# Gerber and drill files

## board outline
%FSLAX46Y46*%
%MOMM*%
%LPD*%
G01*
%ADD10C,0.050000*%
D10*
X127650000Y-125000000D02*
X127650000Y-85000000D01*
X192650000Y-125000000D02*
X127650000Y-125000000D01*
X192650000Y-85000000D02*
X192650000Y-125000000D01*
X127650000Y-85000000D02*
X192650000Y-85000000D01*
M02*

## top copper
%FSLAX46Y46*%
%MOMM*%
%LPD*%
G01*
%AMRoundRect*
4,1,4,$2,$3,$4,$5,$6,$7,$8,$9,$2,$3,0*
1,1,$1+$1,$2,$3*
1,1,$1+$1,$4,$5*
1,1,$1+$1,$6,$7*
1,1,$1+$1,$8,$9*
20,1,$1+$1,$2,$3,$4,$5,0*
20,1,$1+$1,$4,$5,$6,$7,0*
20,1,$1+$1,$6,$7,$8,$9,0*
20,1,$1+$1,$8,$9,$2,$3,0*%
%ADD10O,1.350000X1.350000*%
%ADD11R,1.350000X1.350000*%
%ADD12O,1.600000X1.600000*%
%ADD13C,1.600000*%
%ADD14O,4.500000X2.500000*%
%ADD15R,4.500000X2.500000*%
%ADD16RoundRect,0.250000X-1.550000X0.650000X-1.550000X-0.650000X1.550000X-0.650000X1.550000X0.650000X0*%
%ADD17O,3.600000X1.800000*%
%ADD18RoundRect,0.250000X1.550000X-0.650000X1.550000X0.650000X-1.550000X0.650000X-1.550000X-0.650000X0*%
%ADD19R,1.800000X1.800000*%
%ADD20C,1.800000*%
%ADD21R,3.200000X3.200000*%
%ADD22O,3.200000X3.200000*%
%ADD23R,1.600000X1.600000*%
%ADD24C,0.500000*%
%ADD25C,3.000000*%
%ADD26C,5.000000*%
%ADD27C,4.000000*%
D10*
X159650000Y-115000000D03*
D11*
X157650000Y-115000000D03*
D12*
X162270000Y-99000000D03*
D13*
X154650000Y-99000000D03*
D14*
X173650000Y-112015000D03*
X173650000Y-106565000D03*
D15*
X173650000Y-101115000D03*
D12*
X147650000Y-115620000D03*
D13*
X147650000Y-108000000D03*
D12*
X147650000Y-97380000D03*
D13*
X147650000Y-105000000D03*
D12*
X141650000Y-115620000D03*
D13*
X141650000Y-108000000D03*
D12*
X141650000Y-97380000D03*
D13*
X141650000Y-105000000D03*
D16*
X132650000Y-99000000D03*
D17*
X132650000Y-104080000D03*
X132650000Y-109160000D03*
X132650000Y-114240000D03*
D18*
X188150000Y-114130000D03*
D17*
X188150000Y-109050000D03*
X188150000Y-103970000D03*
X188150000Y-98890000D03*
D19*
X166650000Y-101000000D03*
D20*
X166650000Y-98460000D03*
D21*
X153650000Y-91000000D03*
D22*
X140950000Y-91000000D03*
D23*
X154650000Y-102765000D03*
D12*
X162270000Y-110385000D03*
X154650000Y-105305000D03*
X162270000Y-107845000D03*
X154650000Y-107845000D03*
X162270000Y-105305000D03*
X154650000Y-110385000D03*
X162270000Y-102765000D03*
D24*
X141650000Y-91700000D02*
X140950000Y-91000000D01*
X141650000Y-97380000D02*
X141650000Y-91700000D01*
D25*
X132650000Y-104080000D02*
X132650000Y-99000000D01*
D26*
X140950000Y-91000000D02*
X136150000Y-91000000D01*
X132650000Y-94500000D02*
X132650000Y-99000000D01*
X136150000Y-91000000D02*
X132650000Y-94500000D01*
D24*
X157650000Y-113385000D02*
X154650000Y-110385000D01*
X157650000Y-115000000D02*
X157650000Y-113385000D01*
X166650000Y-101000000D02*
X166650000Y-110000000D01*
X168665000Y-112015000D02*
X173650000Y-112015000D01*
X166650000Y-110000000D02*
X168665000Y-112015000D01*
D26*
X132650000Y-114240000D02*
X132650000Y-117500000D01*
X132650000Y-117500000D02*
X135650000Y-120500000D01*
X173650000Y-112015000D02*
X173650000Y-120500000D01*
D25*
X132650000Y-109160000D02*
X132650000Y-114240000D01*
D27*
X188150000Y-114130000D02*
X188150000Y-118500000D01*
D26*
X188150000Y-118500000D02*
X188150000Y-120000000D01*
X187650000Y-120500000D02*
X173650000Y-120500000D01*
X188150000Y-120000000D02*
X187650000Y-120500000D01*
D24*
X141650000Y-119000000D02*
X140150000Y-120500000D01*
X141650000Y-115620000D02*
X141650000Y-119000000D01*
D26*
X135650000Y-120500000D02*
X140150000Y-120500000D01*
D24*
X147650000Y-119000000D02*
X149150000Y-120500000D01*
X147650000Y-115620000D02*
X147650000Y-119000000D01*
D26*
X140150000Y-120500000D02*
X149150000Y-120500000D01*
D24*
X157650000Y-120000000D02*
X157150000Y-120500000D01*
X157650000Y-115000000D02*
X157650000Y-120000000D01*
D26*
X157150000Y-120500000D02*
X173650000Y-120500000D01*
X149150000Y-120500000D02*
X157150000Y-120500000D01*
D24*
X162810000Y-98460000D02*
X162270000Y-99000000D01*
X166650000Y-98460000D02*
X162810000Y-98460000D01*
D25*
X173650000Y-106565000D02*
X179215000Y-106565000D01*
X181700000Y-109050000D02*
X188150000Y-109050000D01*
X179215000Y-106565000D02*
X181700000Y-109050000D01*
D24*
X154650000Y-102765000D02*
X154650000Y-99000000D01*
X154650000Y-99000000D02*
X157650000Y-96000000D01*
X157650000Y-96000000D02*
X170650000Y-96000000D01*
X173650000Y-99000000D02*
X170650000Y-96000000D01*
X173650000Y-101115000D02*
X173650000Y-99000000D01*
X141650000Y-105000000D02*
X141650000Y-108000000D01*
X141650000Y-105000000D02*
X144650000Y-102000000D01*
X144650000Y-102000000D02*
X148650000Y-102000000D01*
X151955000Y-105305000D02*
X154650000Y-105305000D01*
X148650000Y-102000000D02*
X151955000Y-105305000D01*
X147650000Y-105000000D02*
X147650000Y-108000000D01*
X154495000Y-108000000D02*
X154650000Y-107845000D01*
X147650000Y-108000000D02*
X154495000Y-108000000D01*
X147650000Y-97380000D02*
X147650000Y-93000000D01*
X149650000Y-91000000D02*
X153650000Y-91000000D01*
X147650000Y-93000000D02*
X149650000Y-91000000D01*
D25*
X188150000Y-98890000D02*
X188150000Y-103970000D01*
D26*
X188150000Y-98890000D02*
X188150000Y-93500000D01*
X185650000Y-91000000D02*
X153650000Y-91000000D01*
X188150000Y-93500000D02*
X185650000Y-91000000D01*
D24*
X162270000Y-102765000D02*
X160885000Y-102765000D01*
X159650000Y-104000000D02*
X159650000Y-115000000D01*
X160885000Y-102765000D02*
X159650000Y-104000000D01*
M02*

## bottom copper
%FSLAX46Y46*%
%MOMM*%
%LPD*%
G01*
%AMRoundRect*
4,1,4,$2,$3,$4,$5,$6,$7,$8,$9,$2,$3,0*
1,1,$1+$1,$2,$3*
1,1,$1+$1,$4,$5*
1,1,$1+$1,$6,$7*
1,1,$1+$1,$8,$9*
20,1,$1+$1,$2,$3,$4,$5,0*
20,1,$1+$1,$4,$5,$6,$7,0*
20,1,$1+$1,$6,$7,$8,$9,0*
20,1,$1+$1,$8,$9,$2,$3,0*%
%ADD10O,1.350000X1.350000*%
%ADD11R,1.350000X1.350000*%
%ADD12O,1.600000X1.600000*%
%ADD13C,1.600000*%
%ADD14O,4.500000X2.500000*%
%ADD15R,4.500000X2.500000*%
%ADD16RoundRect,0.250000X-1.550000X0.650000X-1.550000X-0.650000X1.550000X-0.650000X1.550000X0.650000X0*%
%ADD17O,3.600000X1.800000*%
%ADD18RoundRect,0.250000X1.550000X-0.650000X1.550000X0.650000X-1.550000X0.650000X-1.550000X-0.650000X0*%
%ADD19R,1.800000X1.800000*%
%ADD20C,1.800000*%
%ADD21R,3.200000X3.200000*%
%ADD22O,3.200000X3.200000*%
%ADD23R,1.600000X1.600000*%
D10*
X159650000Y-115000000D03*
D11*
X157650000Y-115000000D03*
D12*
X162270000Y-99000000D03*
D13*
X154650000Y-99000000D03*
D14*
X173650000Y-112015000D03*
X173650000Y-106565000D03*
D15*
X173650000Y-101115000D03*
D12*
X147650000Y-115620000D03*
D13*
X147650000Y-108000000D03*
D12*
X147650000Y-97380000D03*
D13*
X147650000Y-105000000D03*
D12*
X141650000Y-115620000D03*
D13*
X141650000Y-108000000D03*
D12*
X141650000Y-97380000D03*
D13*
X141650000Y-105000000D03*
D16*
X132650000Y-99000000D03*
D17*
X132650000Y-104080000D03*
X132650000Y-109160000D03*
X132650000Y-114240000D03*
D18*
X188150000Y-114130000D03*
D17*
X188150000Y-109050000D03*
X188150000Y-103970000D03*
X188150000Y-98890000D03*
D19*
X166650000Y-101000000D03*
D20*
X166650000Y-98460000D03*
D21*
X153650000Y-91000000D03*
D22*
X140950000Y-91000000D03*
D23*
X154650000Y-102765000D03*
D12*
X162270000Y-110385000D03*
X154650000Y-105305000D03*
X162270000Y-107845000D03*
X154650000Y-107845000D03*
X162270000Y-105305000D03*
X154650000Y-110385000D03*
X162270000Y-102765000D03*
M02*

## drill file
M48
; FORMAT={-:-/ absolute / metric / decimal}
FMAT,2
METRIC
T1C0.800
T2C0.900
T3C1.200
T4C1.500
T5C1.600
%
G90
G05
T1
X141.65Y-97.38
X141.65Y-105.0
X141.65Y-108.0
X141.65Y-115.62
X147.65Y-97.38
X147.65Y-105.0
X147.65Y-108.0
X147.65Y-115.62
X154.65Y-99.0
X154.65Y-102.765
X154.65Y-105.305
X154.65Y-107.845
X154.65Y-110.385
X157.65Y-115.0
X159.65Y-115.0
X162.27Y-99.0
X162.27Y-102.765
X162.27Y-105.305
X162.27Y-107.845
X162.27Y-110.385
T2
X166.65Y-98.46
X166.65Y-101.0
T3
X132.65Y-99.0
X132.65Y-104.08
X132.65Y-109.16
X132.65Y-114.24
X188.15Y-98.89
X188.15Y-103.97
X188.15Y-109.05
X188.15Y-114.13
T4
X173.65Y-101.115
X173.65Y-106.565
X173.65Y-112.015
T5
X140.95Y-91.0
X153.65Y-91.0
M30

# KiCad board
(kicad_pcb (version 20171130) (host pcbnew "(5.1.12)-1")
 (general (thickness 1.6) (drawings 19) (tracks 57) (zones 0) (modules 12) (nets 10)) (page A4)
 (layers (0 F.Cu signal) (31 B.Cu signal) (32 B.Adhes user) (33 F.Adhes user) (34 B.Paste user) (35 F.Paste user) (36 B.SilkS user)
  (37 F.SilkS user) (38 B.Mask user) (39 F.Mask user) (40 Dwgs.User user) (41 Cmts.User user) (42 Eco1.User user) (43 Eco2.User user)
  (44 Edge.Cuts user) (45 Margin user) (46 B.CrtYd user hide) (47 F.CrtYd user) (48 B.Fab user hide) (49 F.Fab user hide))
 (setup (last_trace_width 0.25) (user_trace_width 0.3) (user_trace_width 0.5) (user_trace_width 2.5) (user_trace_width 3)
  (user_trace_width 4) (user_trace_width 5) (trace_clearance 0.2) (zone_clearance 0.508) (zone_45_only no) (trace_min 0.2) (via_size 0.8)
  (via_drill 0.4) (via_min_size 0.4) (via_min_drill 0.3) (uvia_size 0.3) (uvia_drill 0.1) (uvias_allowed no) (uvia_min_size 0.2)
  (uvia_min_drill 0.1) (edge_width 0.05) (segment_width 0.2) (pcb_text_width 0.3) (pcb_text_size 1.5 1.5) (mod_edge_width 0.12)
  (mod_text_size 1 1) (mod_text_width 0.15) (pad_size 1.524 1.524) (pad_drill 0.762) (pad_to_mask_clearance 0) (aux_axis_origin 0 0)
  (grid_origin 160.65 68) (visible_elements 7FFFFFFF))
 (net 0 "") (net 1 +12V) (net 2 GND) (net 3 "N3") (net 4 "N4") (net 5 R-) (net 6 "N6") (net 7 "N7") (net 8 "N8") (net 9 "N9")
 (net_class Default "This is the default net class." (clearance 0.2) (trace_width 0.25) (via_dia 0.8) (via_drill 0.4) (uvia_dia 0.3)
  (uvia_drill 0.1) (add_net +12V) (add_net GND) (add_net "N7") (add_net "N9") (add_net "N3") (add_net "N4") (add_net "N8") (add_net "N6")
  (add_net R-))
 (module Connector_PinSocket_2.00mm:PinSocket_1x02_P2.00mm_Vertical (layer F.Cu) (at 157.65 115 90)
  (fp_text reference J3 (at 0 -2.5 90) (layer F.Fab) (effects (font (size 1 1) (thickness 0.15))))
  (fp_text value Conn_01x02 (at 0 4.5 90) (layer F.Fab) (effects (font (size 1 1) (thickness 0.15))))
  (pad 2 thru_hole oval (at 0 2 90) (size 1.35 1.35) (drill 0.8) (layers *.Cu *.Mask) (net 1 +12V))
  (pad 1 thru_hole rect (at 0 0 90) (size 1.35 1.35) (drill 0.8) (layers *.Cu *.Mask) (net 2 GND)))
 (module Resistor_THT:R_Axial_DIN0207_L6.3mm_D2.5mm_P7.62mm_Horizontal (layer F.Cu) (at 154.65 99)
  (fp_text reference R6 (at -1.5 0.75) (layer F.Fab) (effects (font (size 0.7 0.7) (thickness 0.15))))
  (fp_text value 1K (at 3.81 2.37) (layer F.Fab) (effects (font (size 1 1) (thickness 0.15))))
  (pad 2 thru_hole oval (at 7.62 0) (size 1.6 1.6) (drill 0.8) (layers *.Cu *.Mask) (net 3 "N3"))
  (pad 1 thru_hole circle (at 0 0) (size 1.6 1.6) (drill 0.8) (layers *.Cu *.Mask) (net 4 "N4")))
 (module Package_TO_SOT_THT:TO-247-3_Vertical (layer F.Cu) (at 173.65 101.115 270)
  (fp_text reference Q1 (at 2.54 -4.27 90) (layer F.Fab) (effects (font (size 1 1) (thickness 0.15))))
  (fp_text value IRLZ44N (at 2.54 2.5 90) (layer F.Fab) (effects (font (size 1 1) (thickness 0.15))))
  (pad 3 thru_hole oval (at 10.9 0 270) (size 2.5 4.5) (drill 1.5) (layers *.Cu *.Mask) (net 2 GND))
  (pad 2 thru_hole oval (at 5.45 0 270) (size 2.5 4.5) (drill 1.5) (layers *.Cu *.Mask) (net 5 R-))
  (pad 1 thru_hole rect (at 0 0 270) (size 2.5 4.5) (drill 1.5) (layers *.Cu *.Mask) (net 4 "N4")))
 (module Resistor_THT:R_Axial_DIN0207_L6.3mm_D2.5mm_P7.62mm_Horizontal (layer F.Cu) (at 147.65 108 270)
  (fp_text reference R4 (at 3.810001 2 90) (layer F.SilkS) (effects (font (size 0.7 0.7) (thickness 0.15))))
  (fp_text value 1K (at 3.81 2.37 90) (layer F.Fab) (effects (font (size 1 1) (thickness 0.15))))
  (pad 2 thru_hole oval (at 7.62 0 270) (size 1.6 1.6) (drill 0.8) (layers *.Cu *.Mask) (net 2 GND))
  (pad 1 thru_hole circle (at 0 0 270) (size 1.6 1.6) (drill 0.8) (layers *.Cu *.Mask) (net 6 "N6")))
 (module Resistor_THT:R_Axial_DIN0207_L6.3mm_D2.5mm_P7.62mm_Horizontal (layer F.Cu) (at 147.65 105 90)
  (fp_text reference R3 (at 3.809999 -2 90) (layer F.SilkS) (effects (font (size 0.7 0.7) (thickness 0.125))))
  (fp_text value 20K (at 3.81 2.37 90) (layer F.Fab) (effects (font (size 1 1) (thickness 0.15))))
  (pad 2 thru_hole oval (at 7.62 0 90) (size 1.6 1.6) (drill 0.8) (layers *.Cu *.Mask) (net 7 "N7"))
  (pad 1 thru_hole circle (at 0 0 90) (size 1.6 1.6) (drill 0.8) (layers *.Cu *.Mask) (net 6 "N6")))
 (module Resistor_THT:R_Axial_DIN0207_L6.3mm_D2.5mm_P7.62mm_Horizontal (layer F.Cu) (at 141.65 108 270)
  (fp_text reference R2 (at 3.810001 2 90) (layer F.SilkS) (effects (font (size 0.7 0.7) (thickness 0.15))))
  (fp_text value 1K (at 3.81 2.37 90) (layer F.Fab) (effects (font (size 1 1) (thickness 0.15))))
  (pad 2 thru_hole oval (at 7.62 0 270) (size 1.6 1.6) (drill 0.8) (layers *.Cu *.Mask) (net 2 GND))
  (pad 1 thru_hole circle (at 0 0 270) (size 1.6 1.6) (drill 0.8) (layers *.Cu *.Mask) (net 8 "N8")))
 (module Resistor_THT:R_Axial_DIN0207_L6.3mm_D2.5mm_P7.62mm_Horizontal (layer F.Cu) (at 141.65 105 90)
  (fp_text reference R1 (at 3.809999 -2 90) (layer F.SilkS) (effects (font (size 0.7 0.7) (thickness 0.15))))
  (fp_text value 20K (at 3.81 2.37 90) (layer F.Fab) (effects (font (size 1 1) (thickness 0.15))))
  (pad 2 thru_hole oval (at 7.62 0 90) (size 1.6 1.6) (drill 0.8) (layers *.Cu *.Mask) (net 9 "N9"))
  (pad 1 thru_hole circle (at 0 0 90) (size 1.6 1.6) (drill 0.8) (layers *.Cu *.Mask) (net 8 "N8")))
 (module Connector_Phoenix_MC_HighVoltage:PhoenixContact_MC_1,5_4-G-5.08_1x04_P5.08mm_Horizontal (layer F.Cu) (at 132.65 99 270)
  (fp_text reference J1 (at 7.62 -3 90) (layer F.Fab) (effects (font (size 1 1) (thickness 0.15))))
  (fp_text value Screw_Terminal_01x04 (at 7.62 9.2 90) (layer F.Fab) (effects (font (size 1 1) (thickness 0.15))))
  (pad 1 thru_hole roundrect (at 0 0 270) (size 1.8 3.6) (drill 1.2) (layers *.Cu *.Mask) (roundrect_rratio 0.1388888888888889) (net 9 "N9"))
  (pad 2 thru_hole oval (at 5.08 0 270) (size 1.8 3.6) (drill 1.2) (layers *.Cu *.Mask) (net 9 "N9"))
  (pad 3 thru_hole oval (at 10.16 0 270) (size 1.8 3.6) (drill 1.2) (layers *.Cu *.Mask) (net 2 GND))
  (pad 4 thru_hole oval (at 15.24 0 270) (size 1.8 3.6) (drill 1.2) (layers *.Cu *.Mask) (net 2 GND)))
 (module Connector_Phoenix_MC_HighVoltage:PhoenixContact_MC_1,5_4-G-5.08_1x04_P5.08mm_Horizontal (layer F.Cu) (at 188.15 114.13 90)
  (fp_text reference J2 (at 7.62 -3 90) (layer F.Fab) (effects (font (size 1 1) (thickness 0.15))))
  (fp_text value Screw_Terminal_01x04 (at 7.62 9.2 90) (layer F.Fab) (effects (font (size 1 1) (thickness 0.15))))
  (pad 1 thru_hole roundrect (at 0 0 90) (size 1.8 3.6) (drill 1.2) (layers *.Cu *.Mask) (roundrect_rratio 0.1388888888888889) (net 2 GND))
  (pad 2 thru_hole oval (at 5.08 0 90) (size 1.8 3.6) (drill 1.2) (layers *.Cu *.Mask) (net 5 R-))
  (pad 3 thru_hole oval (at 10.16 0 90) (size 1.8 3.6) (drill 1.2) (layers *.Cu *.Mask) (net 7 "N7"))
  (pad 4 thru_hole oval (at 15.24 0 90) (size 1.8 3.6) (drill 1.2) (layers *.Cu *.Mask) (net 7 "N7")))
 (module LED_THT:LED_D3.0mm (layer F.Cu) (at 166.65 101 90)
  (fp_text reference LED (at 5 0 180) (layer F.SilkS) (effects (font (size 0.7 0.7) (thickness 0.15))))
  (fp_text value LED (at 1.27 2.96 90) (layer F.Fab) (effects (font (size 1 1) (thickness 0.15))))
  (pad 1 thru_hole rect (at 0 0 90) (size 1.8 1.8) (drill 0.9) (layers *.Cu *.Mask) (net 2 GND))
  (pad 2 thru_hole circle (at 2.54 0 90) (size 1.8 1.8) (drill 0.9) (layers *.Cu *.Mask) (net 3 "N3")))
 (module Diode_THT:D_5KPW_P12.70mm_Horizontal (layer F.Cu) (at 153.65 91 180)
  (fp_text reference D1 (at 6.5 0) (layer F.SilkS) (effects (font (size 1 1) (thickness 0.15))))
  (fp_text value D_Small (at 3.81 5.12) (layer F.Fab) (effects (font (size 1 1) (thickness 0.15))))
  (pad 1 thru_hole rect (at 0 0 180) (size 3.2 3.2) (drill 1.6) (layers *.Cu *.Mask) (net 7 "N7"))
  (pad 2 thru_hole oval (at 12.7 0 180) (size 3.2 3.2) (drill 1.6) (layers *.Cu *.Mask) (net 9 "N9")))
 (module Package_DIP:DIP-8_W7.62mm (layer F.Cu) (at 154.65 102.765)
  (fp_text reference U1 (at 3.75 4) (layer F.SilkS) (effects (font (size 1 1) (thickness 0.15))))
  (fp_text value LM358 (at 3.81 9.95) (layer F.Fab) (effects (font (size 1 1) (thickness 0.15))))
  (pad 1 thru_hole rect (at 0 0) (size 1.6 1.6) (drill 0.8) (layers *.Cu *.Mask) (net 4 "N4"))
  (pad 5 thru_hole oval (at 7.62 7.62) (size 1.6 1.6) (drill 0.8) (layers *.Cu *.Mask))
  (pad 2 thru_hole oval (at 0 2.54) (size 1.6 1.6) (drill 0.8) (layers *.Cu *.Mask) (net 8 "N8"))
  (pad 6 thru_hole oval (at 7.62 5.08) (size 1.6 1.6) (drill 0.8) (layers *.Cu *.Mask))
  (pad 3 thru_hole oval (at 0 5.08) (size 1.6 1.6) (drill 0.8) (layers *.Cu *.Mask) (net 6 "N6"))
  (pad 7 thru_hole oval (at 7.62 2.54) (size 1.6 1.6) (drill 0.8) (layers *.Cu *.Mask))
  (pad 4 thru_hole oval (at 0 7.62) (size 1.6 1.6) (drill 0.8) (layers *.Cu *.Mask) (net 2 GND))
  (pad 8 thru_hole oval (at 7.62 0) (size 1.6 1.6) (drill 0.8) (layers *.Cu *.Mask) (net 1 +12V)))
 (gr_line (start 127.65 125) (end 127.65 85) (layer Edge.Cuts) (width 0.05))
 (gr_line (start 192.65 125) (end 127.65 125) (layer Edge.Cuts) (width 0.05))
 (gr_line (start 192.65 85) (end 192.65 125) (layer Edge.Cuts) (width 0.05))
 (gr_line (start 127.65 85) (end 192.65 85) (layer Edge.Cuts) (width 0.05))
 (segment (start 141.65 91.7) (end 140.95 91) (width 0.5) (layer F.Cu) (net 9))
 (segment (start 141.65 97.38) (end 141.65 91.7) (width 0.5) (layer F.Cu) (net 9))
 (segment (start 132.65 104.08) (end 132.65 99) (width 3) (layer F.Cu) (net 9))
 (segment (start 140.95 91) (end 136.15 91) (width 5) (layer F.Cu) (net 9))
 (segment (start 132.65 94.5) (end 132.65 99) (width 5) (layer F.Cu) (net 9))
 (segment (start 136.15 91) (end 132.65 94.5) (width 5) (layer F.Cu) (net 9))
 (segment (start 157.65 113.385) (end 154.65 110.385) (width 0.5) (layer F.Cu) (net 2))
 (segment (start 157.65 115) (end 157.65 113.385) (width 0.5) (layer F.Cu) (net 2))
 (segment (start 166.65 101) (end 166.65 110) (width 0.5) (layer F.Cu) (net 2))
 (segment (start 168.665 112.015) (end 173.65 112.015) (width 0.5) (layer F.Cu) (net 2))
 (segment (start 166.65 110) (end 168.665 112.015) (width 0.5) (layer F.Cu) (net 2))
 (segment (start 132.65 114.24) (end 132.65 117.5) (width 5) (layer F.Cu) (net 2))
 (segment (start 132.65 117.5) (end 135.65 120.5) (width 5) (layer F.Cu) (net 2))
 (segment (start 173.65 112.015) (end 173.65 120.5) (width 5) (layer F.Cu) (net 2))
 (segment (start 132.65 109.16) (end 132.65 114.24) (width 3) (layer F.Cu) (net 2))
 (segment (start 188.15 114.13) (end 188.15 118.5) (width 4) (layer F.Cu) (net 2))
 (segment (start 188.15 118.5) (end 188.15 120) (width 5) (layer F.Cu) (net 2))
 (segment (start 187.65 120.5) (end 173.65 120.5) (width 5) (layer F.Cu) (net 2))
 (segment (start 188.15 120) (end 187.65 120.5) (width 5) (layer F.Cu) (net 2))
 (segment (start 141.65 119) (end 140.15 120.5) (width 0.5) (layer F.Cu) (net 2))
 (segment (start 141.65 115.62) (end 141.65 119) (width 0.5) (layer F.Cu) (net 2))
 (segment (start 135.65 120.5) (end 140.15 120.5) (width 5) (layer F.Cu) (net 2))
 (segment (start 147.65 119) (end 149.15 120.5) (width 0.5) (layer F.Cu) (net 2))
 (segment (start 147.65 115.62) (end 147.65 119) (width 0.5) (layer F.Cu) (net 2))
 (segment (start 140.15 120.5) (end 149.15 120.5) (width 5) (layer F.Cu) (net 2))
 (segment (start 157.65 120) (end 157.15 120.5) (width 0.5) (layer F.Cu) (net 2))
 (segment (start 157.65 115) (end 157.65 120) (width 0.5) (layer F.Cu) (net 2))
 (segment (start 157.15 120.5) (end 173.65 120.5) (width 5) (layer F.Cu) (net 2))
 (segment (start 149.15 120.5) (end 157.15 120.5) (width 5) (layer F.Cu) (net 2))
 (segment (start 162.81 98.46) (end 162.27 99) (width 0.5) (layer F.Cu) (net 3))
 (segment (start 166.65 98.46) (end 162.81 98.46) (width 0.5) (layer F.Cu) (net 3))
 (segment (start 173.65 106.565) (end 179.215 106.565) (width 3) (layer F.Cu) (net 5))
 (segment (start 181.7 109.05) (end 188.15 109.05) (width 3) (layer F.Cu) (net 5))
 (segment (start 179.215 106.565) (end 181.7 109.05) (width 3) (layer F.Cu) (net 5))
 (segment (start 154.65 102.765) (end 154.65 99) (width 0.5) (layer F.Cu) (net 4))
 (segment (start 154.65 99) (end 157.65 96) (width 0.5) (layer F.Cu) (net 4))
 (segment (start 157.65 96) (end 170.65 96) (width 0.5) (layer F.Cu) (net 4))
 (segment (start 173.65 99) (end 170.65 96) (width 0.5) (layer F.Cu) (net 4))
 (segment (start 173.65 101.115) (end 173.65 99) (width 0.5) (layer F.Cu) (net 4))
 (segment (start 141.65 105) (end 141.65 108) (width 0.5) (layer F.Cu) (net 8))
 (segment (start 141.65 105) (end 144.65 102) (width 0.5) (layer F.Cu) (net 8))
 (segment (start 144.65 102) (end 148.65 102) (width 0.5) (layer F.Cu) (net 8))
 (segment (start 151.955 105.305) (end 154.65 105.305) (width 0.5) (layer F.Cu) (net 8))
 (segment (start 148.65 102) (end 151.955 105.305) (width 0.5) (layer F.Cu) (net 8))
 (segment (start 147.65 105) (end 147.65 108) (width 0.5) (layer F.Cu) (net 6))
 (segment (start 154.495 108) (end 154.65 107.845) (width 0.5) (layer F.Cu) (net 6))
 (segment (start 147.65 108) (end 154.495 108) (width 0.5) (layer F.Cu) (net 6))
 (segment (start 147.65 97.38) (end 147.65 93) (width 0.5) (layer F.Cu) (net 7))
 (segment (start 149.65 91) (end 153.65 91) (width 0.5) (layer F.Cu) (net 7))
 (segment (start 147.65 93) (end 149.65 91) (width 0.5) (layer F.Cu) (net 7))
 (segment (start 188.15 98.89) (end 188.15 103.97) (width 3) (layer F.Cu) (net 7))
 (segment (start 188.15 98.89) (end 188.15 93.5) (width 5) (layer F.Cu) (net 7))
 (segment (start 185.65 91) (end 153.65 91) (width 5) (layer F.Cu) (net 7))
 (segment (start 188.15 93.5) (end 185.65 91) (width 5) (layer F.Cu) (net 7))
 (segment (start 162.27 102.765) (end 160.885 102.765) (width 0.5) (layer F.Cu) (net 1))
 (segment (start 159.65 104) (end 159.65 115) (width 0.5) (layer F.Cu) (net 1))
 (segment (start 160.885 102.765) (end 159.65 104) (width 0.5) (layer F.Cu) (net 1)))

